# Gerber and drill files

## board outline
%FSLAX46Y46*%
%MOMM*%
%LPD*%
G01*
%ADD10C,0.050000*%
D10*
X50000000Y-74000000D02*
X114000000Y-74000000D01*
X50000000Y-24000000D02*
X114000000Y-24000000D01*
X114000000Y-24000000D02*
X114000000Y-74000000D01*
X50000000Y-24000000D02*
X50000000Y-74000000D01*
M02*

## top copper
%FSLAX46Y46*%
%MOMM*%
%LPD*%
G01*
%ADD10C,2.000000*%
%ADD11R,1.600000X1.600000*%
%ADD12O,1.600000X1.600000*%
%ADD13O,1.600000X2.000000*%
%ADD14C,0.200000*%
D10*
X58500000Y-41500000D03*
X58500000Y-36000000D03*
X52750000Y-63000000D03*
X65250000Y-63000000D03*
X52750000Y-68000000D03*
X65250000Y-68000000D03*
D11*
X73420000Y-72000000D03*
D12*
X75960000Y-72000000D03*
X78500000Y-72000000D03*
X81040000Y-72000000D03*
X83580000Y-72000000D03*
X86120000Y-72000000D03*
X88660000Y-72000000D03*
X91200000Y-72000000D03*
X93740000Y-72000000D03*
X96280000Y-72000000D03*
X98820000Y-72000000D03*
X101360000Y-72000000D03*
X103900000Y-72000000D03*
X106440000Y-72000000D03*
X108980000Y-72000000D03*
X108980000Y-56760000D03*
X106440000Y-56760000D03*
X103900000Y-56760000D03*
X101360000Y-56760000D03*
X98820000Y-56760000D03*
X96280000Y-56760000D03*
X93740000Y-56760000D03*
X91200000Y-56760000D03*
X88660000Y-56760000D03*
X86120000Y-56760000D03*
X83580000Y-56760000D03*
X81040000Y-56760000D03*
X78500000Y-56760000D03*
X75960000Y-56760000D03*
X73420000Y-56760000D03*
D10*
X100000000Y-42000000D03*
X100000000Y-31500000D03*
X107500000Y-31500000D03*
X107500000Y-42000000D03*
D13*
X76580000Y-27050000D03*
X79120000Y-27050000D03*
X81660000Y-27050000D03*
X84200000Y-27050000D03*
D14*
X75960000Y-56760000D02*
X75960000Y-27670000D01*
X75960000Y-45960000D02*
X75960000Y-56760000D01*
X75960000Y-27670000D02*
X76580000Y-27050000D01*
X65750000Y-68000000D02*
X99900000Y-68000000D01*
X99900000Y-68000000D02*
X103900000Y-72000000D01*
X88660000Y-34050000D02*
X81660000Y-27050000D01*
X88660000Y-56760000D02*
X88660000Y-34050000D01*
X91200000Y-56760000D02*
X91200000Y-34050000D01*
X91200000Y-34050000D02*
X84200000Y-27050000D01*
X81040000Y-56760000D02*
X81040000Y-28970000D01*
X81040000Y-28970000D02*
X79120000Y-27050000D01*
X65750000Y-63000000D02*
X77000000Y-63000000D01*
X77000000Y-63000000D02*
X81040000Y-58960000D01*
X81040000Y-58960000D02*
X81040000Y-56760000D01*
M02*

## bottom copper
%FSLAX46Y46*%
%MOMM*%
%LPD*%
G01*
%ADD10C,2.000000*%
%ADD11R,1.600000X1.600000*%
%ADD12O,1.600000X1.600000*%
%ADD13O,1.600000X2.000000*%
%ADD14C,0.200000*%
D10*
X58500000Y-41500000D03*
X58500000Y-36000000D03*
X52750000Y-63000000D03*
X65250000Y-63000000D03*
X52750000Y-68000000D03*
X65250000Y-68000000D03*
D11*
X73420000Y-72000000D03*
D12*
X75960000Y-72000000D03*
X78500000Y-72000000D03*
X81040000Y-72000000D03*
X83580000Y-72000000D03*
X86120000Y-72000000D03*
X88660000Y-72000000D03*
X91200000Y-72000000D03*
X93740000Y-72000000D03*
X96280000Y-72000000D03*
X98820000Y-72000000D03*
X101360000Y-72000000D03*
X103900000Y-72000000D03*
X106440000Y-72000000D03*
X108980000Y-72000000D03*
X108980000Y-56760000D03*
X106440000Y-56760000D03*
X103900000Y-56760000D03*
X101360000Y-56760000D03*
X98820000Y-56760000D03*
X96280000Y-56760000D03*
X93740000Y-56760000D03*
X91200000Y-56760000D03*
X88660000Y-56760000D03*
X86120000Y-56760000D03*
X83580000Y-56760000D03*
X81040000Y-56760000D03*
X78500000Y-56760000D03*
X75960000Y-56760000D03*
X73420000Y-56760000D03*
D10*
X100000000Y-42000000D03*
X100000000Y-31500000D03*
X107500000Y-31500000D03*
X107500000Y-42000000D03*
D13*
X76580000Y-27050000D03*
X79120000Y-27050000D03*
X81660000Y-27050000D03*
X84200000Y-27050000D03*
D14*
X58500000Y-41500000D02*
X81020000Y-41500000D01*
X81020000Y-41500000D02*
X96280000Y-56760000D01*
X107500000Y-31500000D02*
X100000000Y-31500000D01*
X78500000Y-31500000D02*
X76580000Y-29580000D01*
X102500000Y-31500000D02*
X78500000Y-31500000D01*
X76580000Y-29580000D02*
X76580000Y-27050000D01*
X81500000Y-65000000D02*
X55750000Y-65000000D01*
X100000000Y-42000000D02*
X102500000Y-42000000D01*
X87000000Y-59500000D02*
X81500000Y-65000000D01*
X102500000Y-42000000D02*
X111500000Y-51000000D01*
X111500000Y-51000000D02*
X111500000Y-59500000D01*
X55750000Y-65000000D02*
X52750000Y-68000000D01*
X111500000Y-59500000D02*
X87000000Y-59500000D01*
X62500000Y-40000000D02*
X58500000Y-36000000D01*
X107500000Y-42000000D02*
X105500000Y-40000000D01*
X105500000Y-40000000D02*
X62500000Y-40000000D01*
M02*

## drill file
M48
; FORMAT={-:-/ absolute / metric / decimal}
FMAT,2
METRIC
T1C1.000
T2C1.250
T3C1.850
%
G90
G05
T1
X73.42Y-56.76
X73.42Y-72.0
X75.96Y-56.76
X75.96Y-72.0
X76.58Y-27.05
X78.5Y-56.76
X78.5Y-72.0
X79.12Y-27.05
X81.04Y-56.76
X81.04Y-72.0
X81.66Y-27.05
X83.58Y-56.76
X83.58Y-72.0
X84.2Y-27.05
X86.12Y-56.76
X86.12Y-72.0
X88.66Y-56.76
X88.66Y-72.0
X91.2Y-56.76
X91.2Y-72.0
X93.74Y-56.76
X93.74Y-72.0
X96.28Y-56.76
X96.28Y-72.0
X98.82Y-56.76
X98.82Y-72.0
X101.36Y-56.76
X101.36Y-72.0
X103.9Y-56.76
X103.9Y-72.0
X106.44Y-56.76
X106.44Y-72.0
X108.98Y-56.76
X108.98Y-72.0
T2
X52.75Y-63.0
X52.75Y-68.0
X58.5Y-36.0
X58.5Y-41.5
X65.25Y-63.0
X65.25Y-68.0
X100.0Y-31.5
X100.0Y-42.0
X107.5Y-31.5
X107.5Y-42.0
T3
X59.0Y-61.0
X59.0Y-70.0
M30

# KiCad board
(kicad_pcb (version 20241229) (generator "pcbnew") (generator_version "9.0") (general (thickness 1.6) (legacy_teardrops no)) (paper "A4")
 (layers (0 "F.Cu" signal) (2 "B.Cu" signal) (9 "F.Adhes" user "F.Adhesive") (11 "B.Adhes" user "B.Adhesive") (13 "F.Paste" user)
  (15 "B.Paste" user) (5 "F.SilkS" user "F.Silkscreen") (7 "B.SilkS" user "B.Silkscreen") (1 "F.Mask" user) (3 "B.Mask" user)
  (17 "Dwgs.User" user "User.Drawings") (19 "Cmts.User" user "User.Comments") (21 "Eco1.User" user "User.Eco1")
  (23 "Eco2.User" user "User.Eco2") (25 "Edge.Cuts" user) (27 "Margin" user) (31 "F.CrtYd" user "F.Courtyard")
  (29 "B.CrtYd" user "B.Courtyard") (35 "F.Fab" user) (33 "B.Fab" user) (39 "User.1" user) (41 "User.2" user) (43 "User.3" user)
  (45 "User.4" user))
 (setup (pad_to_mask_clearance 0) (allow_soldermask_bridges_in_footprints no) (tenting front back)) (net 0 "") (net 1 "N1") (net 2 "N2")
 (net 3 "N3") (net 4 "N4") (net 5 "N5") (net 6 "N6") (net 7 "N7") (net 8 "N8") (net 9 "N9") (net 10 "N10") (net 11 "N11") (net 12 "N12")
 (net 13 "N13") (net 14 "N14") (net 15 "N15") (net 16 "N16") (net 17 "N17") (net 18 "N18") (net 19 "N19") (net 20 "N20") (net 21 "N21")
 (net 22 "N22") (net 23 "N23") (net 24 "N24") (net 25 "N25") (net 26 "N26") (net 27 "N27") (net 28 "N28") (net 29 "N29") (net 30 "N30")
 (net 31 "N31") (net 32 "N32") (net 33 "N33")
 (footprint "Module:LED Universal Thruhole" (layer "F.Cu") (at 58.5 38.5 90)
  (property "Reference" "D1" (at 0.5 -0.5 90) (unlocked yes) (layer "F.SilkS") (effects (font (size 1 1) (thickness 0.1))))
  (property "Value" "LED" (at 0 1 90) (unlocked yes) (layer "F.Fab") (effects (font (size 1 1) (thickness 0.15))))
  (pad "1" thru_hole circle (at -3 0 270) (size 2 2) (drill 1.25) (layers "*.Cu" "*.Mask") (remove_unused_layers no) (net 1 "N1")
   (solder_mask_margin 0.102))
  (pad "2" thru_hole circle (at 2.5 0 270) (size 2 2) (drill 1.25) (layers "*.Cu" "*.Mask") (remove_unused_layers no) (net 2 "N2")
   (solder_mask_margin 0.102)))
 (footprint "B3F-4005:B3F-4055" (layer "F.Cu") (at 59 65.5 180)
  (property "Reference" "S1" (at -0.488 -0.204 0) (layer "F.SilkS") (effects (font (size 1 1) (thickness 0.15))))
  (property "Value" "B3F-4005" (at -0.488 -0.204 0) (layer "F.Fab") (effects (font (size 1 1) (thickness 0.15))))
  (pad "" np_thru_hole circle (at 0 -4.5 180) (size 1.85 1.85) (drill 1.85) (layers "*.Cu" "*.Mask"))
  (pad "" np_thru_hole circle (at 0 4.5 180) (size 1.85 1.85) (drill 1.85) (layers "*.Cu" "*.Mask"))
  (pad "1" thru_hole circle (at 6.25 2.5 180) (size 2 2) (drill 1.25) (layers "*.Cu" "*.Mask") (remove_unused_layers no) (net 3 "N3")
   (solder_mask_margin 0.102))
  (pad "2" thru_hole circle (at -6.25 2.5 180) (size 2 2) (drill 1.25) (layers "*.Cu" "*.Mask") (remove_unused_layers no) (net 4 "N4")
   (solder_mask_margin 0.102))
  (pad "3" thru_hole circle (at 6.25 -2.5 180) (size 2 2) (drill 1.25) (layers "*.Cu" "*.Mask") (remove_unused_layers no) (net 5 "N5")
   (solder_mask_margin 0.102))
  (pad "4" thru_hole circle (at -6.25 -2.5 180) (size 2 2) (drill 1.25) (layers "*.Cu" "*.Mask") (remove_unused_layers no) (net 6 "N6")
   (solder_mask_margin 0.102)))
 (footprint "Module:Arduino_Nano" (layer "F.Cu") (at 73.42 72 90)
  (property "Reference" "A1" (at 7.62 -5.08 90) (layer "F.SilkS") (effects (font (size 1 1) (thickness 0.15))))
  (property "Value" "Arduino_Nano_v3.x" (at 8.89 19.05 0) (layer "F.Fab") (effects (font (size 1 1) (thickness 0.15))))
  (pad "1" thru_hole rect (at 0 0 90) (size 1.6 1.6) (drill 1) (layers "*.Cu" "*.Mask") (remove_unused_layers no) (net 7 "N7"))
  (pad "2" thru_hole oval (at 0 2.54 90) (size 1.6 1.6) (drill 1) (layers "*.Cu" "*.Mask") (remove_unused_layers no) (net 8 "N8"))
  (pad "3" thru_hole oval (at 0 5.08 90) (size 1.6 1.6) (drill 1) (layers "*.Cu" "*.Mask") (remove_unused_layers no) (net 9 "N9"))
  (pad "4" thru_hole oval (at 0 7.62 90) (size 1.6 1.6) (drill 1) (layers "*.Cu" "*.Mask") (remove_unused_layers no) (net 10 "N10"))
  (pad "5" thru_hole oval (at 0 10.16 90) (size 1.6 1.6) (drill 1) (layers "*.Cu" "*.Mask") (remove_unused_layers no) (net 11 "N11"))
  (pad "6" thru_hole oval (at 0 12.7 90) (size 1.6 1.6) (drill 1) (layers "*.Cu" "*.Mask") (remove_unused_layers no) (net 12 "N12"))
  (pad "7" thru_hole oval (at 0 15.24 90) (size 1.6 1.6) (drill 1) (layers "*.Cu" "*.Mask") (remove_unused_layers no) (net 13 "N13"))
  (pad "8" thru_hole oval (at 0 17.78 90) (size 1.6 1.6) (drill 1) (layers "*.Cu" "*.Mask") (remove_unused_layers no) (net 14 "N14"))
  (pad "9" thru_hole oval (at 0 20.32 90) (size 1.6 1.6) (drill 1) (layers "*.Cu" "*.Mask") (remove_unused_layers no) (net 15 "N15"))
  (pad "10" thru_hole oval (at 0 22.86 90) (size 1.6 1.6) (drill 1) (layers "*.Cu" "*.Mask") (remove_unused_layers no) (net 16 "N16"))
  (pad "11" thru_hole oval (at 0 25.4 90) (size 1.6 1.6) (drill 1) (layers "*.Cu" "*.Mask") (remove_unused_layers no) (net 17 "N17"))
  (pad "12" thru_hole oval (at 0 27.94 90) (size 1.6 1.6) (drill 1) (layers "*.Cu" "*.Mask") (remove_unused_layers no) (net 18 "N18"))
  (pad "13" thru_hole oval (at 0 30.48 90) (size 1.6 1.6) (drill 1) (layers "*.Cu" "*.Mask") (remove_unused_layers no) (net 6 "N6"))
  (pad "14" thru_hole oval (at 0 33.02 90) (size 1.6 1.6) (drill 1) (layers "*.Cu" "*.Mask") (remove_unused_layers no) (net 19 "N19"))
  (pad "15" thru_hole oval (at 0 35.56 90) (size 1.6 1.6) (drill 1) (layers "*.Cu" "*.Mask") (remove_unused_layers no) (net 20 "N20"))
  (pad "16" thru_hole oval (at 15.24 35.56 90) (size 1.6 1.6) (drill 1) (layers "*.Cu" "*.Mask") (remove_unused_layers no) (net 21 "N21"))
  (pad "17" thru_hole oval (at 15.24 33.02 90) (size 1.6 1.6) (drill 1) (layers "*.Cu" "*.Mask") (remove_unused_layers no) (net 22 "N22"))
  (pad "18" thru_hole oval (at 15.24 30.48 90) (size 1.6 1.6) (drill 1) (layers "*.Cu" "*.Mask") (remove_unused_layers no) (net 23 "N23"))
  (pad "19" thru_hole oval (at 15.24 27.94 90) (size 1.6 1.6) (drill 1) (layers "*.Cu" "*.Mask") (remove_unused_layers no) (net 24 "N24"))
  (pad "20" thru_hole oval (at 15.24 25.4 90) (size 1.6 1.6) (drill 1) (layers "*.Cu" "*.Mask") (remove_unused_layers no) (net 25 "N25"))
  (pad "21" thru_hole oval (at 15.24 22.86 90) (size 1.6 1.6) (drill 1) (layers "*.Cu" "*.Mask") (remove_unused_layers no) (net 1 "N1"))
  (pad "22" thru_hole oval (at 15.24 20.32 90) (size 1.6 1.6) (drill 1) (layers "*.Cu" "*.Mask") (remove_unused_layers no) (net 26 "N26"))
  (pad "23" thru_hole oval (at 15.24 17.78 90) (size 1.6 1.6) (drill 1) (layers "*.Cu" "*.Mask") (remove_unused_layers no) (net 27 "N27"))
  (pad "24" thru_hole oval (at 15.24 15.24 90) (size 1.6 1.6) (drill 1) (layers "*.Cu" "*.Mask") (remove_unused_layers no) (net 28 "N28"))
  (pad "25" thru_hole oval (at 15.24 12.7 90) (size 1.6 1.6) (drill 1) (layers "*.Cu" "*.Mask") (remove_unused_layers no) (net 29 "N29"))
  (pad "26" thru_hole oval (at 15.24 10.16 90) (size 1.6 1.6) (drill 1) (layers "*.Cu" "*.Mask") (remove_unused_layers no) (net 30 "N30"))
  (pad "27" thru_hole oval (at 15.24 7.62 90) (size 1.6 1.6) (drill 1) (layers "*.Cu" "*.Mask") (remove_unused_layers no) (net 4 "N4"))
  (pad "28" thru_hole oval (at 15.24 5.08 90) (size 1.6 1.6) (drill 1) (layers "*.Cu" "*.Mask") (remove_unused_layers no) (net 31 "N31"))
  (pad "29" thru_hole oval (at 15.24 2.54 90) (size 1.6 1.6) (drill 1) (layers "*.Cu" "*.Mask") (remove_unused_layers no) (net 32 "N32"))
  (pad "30" thru_hole oval (at 15.24 0 90) (size 1.6 1.6) (drill 1) (layers "*.Cu" "*.Mask") (remove_unused_layers no) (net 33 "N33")))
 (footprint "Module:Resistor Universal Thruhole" (layer "F.Cu") (at 100 36.5 90)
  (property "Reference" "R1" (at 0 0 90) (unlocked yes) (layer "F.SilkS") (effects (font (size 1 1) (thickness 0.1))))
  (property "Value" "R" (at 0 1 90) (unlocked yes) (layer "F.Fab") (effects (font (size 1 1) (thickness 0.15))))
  (pad "1" thru_hole circle (at -5.5 0 270) (size 2 2) (drill 1.25) (layers "*.Cu" "*.Mask") (remove_unused_layers no) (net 5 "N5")
   (solder_mask_margin 0.102))
  (pad "2" thru_hole circle (at 5 0 270) (size 2 2) (drill 1.25) (layers "*.Cu" "*.Mask") (remove_unused_layers no) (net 32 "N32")
   (solder_mask_margin 0.102)))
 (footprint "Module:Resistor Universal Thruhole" (layer "F.Cu") (at 107.5 37 -90)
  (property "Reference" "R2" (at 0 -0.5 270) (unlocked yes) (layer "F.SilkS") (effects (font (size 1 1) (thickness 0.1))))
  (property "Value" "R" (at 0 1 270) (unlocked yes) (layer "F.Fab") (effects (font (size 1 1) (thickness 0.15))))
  (pad "1" thru_hole circle (at -5.5 0 90) (size 2 2) (drill 1.25) (layers "*.Cu" "*.Mask") (remove_unused_layers no) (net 32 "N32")
   (solder_mask_margin 0.102))
  (pad "2" thru_hole circle (at 5 0 90) (size 2 2) (drill 1.25) (layers "*.Cu" "*.Mask") (remove_unused_layers no) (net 2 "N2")
   (solder_mask_margin 0.102)))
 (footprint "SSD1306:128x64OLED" (layer "F.Cu") (at 80.2 37.65)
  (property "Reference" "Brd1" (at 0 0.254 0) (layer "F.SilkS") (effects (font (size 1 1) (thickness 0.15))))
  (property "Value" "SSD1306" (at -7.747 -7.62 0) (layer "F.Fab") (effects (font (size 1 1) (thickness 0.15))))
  (pad "1" thru_hole oval (at -3.62 -10.6 90) (size 2 1.6) (drill 1) (layers "*.Cu" "*.Mask") (remove_unused_layers no) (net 32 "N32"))
  (pad "2" thru_hole oval (at -1.08 -10.6 90) (size 2 1.6) (drill 1) (layers "*.Cu" "*.Mask") (remove_unused_layers no) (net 4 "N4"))
  (pad "3" thru_hole oval (at 1.46 -10.6 90) (size 2 1.6) (drill 1) (layers "*.Cu" "*.Mask") (remove_unused_layers no) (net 28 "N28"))
  (pad "4" thru_hole oval (at 4 -10.6 90) (size 2 1.6) (drill 1) (layers "*.Cu" "*.Mask") (remove_unused_layers no) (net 27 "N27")))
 (gr_line (start 50 74) (end 114 74) (stroke (width 0.05) (type default)) (layer "Edge.Cuts"))
 (gr_line (start 50 24) (end 114 24) (stroke (width 0.05) (type default)) (layer "Edge.Cuts"))
 (gr_line (start 114 24) (end 114 74) (stroke (width 0.05) (type default)) (layer "Edge.Cuts"))
 (gr_line (start 50 24) (end 50 74) (stroke (width 0.05) (type default)) (layer "Edge.Cuts"))
 (segment (start 58.5 41.5) (end 81.02 41.5) (width 0.2) (layer "B.Cu") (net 1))
 (segment (start 81.02 41.5) (end 96.28 56.76) (width 0.2) (layer "B.Cu") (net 1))
 (segment (start 75.96 56.76) (end 75.96 27.67) (width 0.2) (layer "F.Cu") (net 32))
 (segment (start 75.96 45.96) (end 75.96 56.76) (width 0.2) (layer "F.Cu") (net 32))
 (segment (start 75.96 27.67) (end 76.58 27.05) (width 0.2) (layer "F.Cu") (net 32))
 (segment (start 107.5 31.5) (end 100 31.5) (width 0.2) (layer "B.Cu") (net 32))
 (segment (start 78.5 31.5) (end 76.58 29.58) (width 0.2) (layer "B.Cu") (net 32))
 (segment (start 102.5 31.5) (end 78.5 31.5) (width 0.2) (layer "B.Cu") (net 32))
 (segment (start 76.58 29.58) (end 76.58 27.05) (width 0.2) (layer "B.Cu") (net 32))
 (segment (start 65.75 68) (end 99.9 68) (width 0.2) (layer "F.Cu") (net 6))
 (segment (start 99.9 68) (end 103.9 72) (width 0.2) (layer "F.Cu") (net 6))
 (segment (start 88.66 34.05) (end 81.66 27.05) (width 0.2) (layer "F.Cu") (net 28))
 (segment (start 88.66 56.76) (end 88.66 34.05) (width 0.2) (layer "F.Cu") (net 28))
 (segment (start 91.2 56.76) (end 91.2 34.05) (width 0.2) (layer "F.Cu") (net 27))
 (segment (start 91.2 34.05) (end 84.2 27.05) (width 0.2) (layer "F.Cu") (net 27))
 (segment (start 81.04 56.76) (end 81.04 28.97) (width 0.2) (layer "F.Cu") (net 4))
 (segment (start 81.04 28.97) (end 79.12 27.05) (width 0.2) (layer "F.Cu") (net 4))
 (segment (start 65.75 63) (end 77 63) (width 0.2) (layer "F.Cu") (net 4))
 (segment (start 77 63) (end 81.04 58.96) (width 0.2) (layer "F.Cu") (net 4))
 (segment (start 81.04 58.96) (end 81.04 56.76) (width 0.2) (layer "F.Cu") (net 4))
 (segment (start 81.5 65) (end 55.75 65) (width 0.2) (layer "B.Cu") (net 5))
 (segment (start 100 42) (end 102.5 42) (width 0.2) (layer "B.Cu") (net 5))
 (segment (start 87 59.5) (end 81.5 65) (width 0.2) (layer "B.Cu") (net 5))
 (segment (start 102.5 42) (end 111.5 51) (width 0.2) (layer "B.Cu") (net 5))
 (segment (start 111.5 51) (end 111.5 59.5) (width 0.2) (layer "B.Cu") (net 5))
 (segment (start 55.75 65) (end 52.75 68) (width 0.2) (layer "B.Cu") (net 5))
 (segment (start 111.5 59.5) (end 87 59.5) (width 0.2) (layer "B.Cu") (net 5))
 (segment (start 62.5 40) (end 58.5 36) (width 0.2) (layer "B.Cu") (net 2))
 (segment (start 107.5 42) (end 105.5 40) (width 0.2) (layer "B.Cu") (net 2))
 (segment (start 105.5 40) (end 62.5 40) (width 0.2) (layer "B.Cu") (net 2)))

